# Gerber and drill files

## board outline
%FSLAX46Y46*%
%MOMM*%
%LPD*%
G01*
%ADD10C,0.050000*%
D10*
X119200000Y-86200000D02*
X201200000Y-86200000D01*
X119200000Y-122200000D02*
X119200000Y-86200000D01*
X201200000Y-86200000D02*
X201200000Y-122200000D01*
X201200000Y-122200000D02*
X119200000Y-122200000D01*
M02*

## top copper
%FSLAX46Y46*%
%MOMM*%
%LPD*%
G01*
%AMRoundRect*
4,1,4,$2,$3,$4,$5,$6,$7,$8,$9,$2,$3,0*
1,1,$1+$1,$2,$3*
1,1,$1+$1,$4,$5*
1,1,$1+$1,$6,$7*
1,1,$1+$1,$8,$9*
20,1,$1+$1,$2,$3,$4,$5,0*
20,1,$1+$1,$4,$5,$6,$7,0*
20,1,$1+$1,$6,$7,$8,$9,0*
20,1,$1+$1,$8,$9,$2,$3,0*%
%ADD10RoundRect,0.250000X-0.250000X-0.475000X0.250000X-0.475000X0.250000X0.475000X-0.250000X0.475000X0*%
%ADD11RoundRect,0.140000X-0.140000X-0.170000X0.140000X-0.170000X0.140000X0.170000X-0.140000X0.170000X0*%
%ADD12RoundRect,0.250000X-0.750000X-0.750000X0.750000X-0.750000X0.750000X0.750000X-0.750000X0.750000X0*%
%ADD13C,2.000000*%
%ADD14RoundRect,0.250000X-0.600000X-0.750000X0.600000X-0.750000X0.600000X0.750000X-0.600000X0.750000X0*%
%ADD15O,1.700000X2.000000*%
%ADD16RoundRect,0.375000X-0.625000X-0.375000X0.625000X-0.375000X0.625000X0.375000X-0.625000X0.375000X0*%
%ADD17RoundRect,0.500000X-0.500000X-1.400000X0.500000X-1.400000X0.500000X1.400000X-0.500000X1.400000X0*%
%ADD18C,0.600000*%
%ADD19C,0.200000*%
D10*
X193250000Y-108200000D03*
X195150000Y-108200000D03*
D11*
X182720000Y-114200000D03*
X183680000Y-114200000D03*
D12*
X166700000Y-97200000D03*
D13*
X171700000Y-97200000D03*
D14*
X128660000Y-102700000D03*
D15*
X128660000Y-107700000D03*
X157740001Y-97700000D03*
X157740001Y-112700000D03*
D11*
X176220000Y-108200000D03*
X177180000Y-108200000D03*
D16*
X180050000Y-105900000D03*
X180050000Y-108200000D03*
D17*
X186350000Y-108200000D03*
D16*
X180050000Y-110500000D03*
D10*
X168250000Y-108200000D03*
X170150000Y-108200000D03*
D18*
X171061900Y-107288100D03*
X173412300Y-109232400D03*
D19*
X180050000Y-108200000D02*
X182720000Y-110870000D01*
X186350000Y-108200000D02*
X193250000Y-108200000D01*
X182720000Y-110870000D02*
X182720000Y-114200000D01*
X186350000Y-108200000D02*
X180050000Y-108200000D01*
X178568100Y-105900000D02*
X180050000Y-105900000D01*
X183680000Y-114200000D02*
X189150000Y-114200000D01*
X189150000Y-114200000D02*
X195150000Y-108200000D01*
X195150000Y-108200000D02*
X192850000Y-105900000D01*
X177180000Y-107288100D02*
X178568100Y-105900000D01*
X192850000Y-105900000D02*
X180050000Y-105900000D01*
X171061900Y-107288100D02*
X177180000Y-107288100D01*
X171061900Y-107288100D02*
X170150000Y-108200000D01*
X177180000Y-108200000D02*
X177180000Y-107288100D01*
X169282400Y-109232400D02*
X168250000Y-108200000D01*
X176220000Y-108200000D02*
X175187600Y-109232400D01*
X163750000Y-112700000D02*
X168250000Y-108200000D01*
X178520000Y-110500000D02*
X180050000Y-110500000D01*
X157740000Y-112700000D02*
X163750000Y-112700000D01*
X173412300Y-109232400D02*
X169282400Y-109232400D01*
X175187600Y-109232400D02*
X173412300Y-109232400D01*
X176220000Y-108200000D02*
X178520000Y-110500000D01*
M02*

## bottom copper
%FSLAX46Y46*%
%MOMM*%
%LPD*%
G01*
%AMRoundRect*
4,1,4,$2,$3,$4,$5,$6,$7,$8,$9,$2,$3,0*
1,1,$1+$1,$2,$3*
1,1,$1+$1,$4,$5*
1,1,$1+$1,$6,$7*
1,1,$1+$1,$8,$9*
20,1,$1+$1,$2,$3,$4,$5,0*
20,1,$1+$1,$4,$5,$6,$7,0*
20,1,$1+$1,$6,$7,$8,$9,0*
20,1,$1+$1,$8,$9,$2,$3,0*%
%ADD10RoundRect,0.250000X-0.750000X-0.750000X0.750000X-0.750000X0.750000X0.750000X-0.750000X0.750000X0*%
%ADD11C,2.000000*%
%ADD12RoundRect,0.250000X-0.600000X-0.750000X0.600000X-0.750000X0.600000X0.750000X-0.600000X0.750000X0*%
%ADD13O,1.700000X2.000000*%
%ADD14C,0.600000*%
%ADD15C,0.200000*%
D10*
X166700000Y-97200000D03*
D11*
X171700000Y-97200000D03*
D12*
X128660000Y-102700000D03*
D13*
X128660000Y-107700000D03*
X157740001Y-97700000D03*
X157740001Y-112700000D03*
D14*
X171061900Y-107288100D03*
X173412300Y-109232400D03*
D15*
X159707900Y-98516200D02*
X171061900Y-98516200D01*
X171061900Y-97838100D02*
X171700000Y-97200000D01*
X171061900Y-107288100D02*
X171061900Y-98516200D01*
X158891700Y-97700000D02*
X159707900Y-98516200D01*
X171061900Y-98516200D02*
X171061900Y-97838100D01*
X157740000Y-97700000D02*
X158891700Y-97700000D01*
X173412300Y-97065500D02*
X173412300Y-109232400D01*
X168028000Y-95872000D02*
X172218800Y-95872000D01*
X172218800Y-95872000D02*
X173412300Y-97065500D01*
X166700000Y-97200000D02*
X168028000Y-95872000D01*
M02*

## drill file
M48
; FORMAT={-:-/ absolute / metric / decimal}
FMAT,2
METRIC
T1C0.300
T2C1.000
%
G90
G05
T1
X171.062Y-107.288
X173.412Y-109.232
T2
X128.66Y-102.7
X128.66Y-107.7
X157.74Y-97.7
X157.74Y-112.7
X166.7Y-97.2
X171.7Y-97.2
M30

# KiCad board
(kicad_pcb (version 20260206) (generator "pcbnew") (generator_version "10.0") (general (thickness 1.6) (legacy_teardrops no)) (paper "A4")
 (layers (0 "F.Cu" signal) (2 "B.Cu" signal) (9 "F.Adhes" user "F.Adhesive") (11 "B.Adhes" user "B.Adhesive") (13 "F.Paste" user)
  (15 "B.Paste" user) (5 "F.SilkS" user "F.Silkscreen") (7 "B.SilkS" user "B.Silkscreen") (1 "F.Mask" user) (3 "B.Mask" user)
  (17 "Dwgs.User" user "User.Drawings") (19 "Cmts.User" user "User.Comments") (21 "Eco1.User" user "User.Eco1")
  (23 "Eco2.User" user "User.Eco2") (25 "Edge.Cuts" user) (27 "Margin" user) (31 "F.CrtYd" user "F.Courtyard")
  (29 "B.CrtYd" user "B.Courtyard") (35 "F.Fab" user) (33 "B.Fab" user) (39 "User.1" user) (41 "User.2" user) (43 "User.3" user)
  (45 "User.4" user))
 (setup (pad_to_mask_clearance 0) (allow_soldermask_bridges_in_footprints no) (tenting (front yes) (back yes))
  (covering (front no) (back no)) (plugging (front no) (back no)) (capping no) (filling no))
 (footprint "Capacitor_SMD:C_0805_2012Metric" (layer "F.Cu") (at 194.2 108.2)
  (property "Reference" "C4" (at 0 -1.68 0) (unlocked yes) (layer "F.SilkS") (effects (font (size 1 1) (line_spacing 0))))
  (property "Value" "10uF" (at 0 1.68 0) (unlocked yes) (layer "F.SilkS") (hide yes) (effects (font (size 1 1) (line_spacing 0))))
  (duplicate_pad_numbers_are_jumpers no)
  (pad "1" smd roundrect (at -0.95 0) (size 1 1.45) (layers "F.Cu" "F.Mask" "F.Paste") (roundrect_rratio 0.25) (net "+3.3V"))
  (pad "2" smd roundrect (at 0.95 0) (size 1 1.45) (layers "F.Cu" "F.Mask" "F.Paste") (roundrect_rratio 0.25) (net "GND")))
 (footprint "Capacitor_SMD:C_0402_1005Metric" (layer "F.Cu") (at 183.2 114.2)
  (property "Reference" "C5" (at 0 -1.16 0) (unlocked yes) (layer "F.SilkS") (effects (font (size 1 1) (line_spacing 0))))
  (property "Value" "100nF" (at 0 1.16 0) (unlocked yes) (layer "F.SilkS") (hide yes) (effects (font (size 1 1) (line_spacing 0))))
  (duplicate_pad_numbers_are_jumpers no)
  (pad "1" smd roundrect (at -0.48 0) (size 0.56 0.62) (layers "F.Cu" "F.Mask" "F.Paste") (roundrect_rratio 0.25) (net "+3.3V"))
  (pad "2" smd roundrect (at 0.48 0) (size 0.56 0.62) (layers "F.Cu" "F.Mask" "F.Paste") (roundrect_rratio 0.25) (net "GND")))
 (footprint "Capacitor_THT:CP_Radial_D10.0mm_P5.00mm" (layer "F.Cu") (at 166.7 97.2)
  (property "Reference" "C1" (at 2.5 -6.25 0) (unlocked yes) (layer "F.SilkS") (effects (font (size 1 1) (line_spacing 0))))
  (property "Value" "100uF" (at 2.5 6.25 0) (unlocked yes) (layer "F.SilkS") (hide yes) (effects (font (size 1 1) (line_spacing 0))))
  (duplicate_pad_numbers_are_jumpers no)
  (pad "1" thru_hole roundrect (at 0 0) (size 2 2) (drill 1) (layers "*.Cu" "*.Mask") (remove_unused_layers no) (roundrect_rratio 0.125)
   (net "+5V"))
  (pad "2" thru_hole circle (at 5 0) (size 2 2) (drill 1) (layers "*.Cu" "*.Mask") (remove_unused_layers no) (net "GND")))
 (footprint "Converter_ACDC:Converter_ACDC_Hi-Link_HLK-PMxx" (layer "F.Cu") (at 128.66 102.7)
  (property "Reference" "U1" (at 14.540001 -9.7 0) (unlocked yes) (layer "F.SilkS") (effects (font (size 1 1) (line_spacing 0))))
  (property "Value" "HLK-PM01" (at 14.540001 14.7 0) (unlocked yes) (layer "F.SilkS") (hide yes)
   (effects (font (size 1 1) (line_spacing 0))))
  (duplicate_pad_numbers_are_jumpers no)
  (pad "1" thru_hole roundrect (at 0 0) (size 1.7 2) (drill 1) (layers "*.Cu" "*.Mask") (remove_unused_layers no)
   (roundrect_rratio 0.147059) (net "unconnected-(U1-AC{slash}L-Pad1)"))
  (pad "2" thru_hole oval (at 0 5) (size 1.7 2) (drill 1) (layers "*.Cu" "*.Mask") (remove_unused_layers no)
   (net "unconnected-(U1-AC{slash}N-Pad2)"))
  (pad "3" thru_hole oval (at 29.080001 -5) (size 1.7 2) (drill 1) (layers "*.Cu" "*.Mask") (remove_unused_layers no) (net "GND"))
  (pad "4" thru_hole oval (at 29.080001 10) (size 1.7 2) (drill 1) (layers "*.Cu" "*.Mask") (remove_unused_layers no) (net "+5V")))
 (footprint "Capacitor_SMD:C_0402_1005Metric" (layer "F.Cu") (at 176.7 108.2)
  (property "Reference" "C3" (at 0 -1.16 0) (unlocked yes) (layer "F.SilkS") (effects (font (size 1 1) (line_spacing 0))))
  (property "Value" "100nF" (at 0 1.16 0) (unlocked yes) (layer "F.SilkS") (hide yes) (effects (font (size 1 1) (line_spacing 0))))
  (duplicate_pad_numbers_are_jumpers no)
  (pad "1" smd roundrect (at -0.48 0) (size 0.56 0.62) (layers "F.Cu" "F.Mask" "F.Paste") (roundrect_rratio 0.25) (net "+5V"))
  (pad "2" smd roundrect (at 0.48 0) (size 0.56 0.62) (layers "F.Cu" "F.Mask" "F.Paste") (roundrect_rratio 0.25) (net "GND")))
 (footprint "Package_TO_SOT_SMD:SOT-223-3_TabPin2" (layer "F.Cu") (at 183.2 108.2)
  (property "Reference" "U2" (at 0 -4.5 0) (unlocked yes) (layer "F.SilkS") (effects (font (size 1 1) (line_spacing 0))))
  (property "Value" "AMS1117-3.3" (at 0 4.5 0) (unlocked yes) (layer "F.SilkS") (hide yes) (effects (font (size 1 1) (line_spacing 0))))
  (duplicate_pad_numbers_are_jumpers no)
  (pad "1" smd roundrect (at -3.15 -2.3) (size 2 1.5) (layers "F.Cu" "F.Mask" "F.Paste") (roundrect_rratio 0.25) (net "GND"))
  (pad "2" smd roundrect (at -3.15 0) (size 2 1.5) (layers "F.Cu" "F.Mask" "F.Paste") (roundrect_rratio 0.25) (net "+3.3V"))
  (pad "2" smd roundrect (at 3.15 0) (size 2 3.8) (layers "F.Cu" "F.Mask" "F.Paste") (roundrect_rratio 0.25) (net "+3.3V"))
  (pad "3" smd roundrect (at -3.15 2.3) (size 2 1.5) (layers "F.Cu" "F.Mask" "F.Paste") (roundrect_rratio 0.25) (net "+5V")))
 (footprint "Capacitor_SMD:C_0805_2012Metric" (layer "F.Cu") (at 169.2 108.2)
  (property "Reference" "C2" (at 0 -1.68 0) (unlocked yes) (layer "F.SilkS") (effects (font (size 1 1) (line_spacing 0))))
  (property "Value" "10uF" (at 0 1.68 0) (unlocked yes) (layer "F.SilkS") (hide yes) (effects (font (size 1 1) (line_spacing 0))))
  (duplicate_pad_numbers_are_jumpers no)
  (pad "1" smd roundrect (at -0.95 0) (size 1 1.45) (layers "F.Cu" "F.Mask" "F.Paste") (roundrect_rratio 0.25) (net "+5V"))
  (pad "2" smd roundrect (at 0.95 0) (size 1 1.45) (layers "F.Cu" "F.Mask" "F.Paste") (roundrect_rratio 0.25) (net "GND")))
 (gr_line (start 119.2 86.2) (end 201.2 86.2) (stroke (width 0.05) (type default)) (layer "Edge.Cuts"))
 (gr_line (start 119.2 122.2) (end 119.2 86.2) (stroke (width 0.05) (type default)) (layer "Edge.Cuts"))
 (gr_line (start 201.2 86.2) (end 201.2 122.2) (stroke (width 0.05) (type default)) (layer "Edge.Cuts"))
 (gr_line (start 201.2 122.2) (end 119.2 122.2) (stroke (width 0.05) (type default)) (layer "Edge.Cuts"))
 (segment (start 180.05 108.2) (end 182.72 110.87) (width 0.2) (layer "F.Cu") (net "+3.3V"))
 (segment (start 186.35 108.2) (end 193.25 108.2) (width 0.2) (layer "F.Cu") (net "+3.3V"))
 (segment (start 182.72 110.87) (end 182.72 114.2) (width 0.2) (layer "F.Cu") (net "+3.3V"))
 (segment (start 186.35 108.2) (end 180.05 108.2) (width 0.2) (layer "F.Cu") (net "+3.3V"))
 (segment (start 178.5681 105.9) (end 180.05 105.9) (width 0.2) (layer "F.Cu") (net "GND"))
 (segment (start 183.68 114.2) (end 189.15 114.2) (width 0.2) (layer "F.Cu") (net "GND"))
 (segment (start 189.15 114.2) (end 195.15 108.2) (width 0.2) (layer "F.Cu") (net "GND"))
 (segment (start 195.15 108.2) (end 192.85 105.9) (width 0.2) (layer "F.Cu") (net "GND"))
 (segment (start 177.18 107.2881) (end 178.5681 105.9) (width 0.2) (layer "F.Cu") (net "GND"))
 (segment (start 192.85 105.9) (end 180.05 105.9) (width 0.2) (layer "F.Cu") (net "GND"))
 (segment (start 171.0619 107.2881) (end 177.18 107.2881) (width 0.2) (layer "F.Cu") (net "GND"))
 (segment (start 171.0619 107.2881) (end 170.15 108.2) (width 0.2) (layer "F.Cu") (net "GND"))
 (segment (start 177.18 108.2) (end 177.18 107.2881) (width 0.2) (layer "F.Cu") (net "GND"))
 (via (at 171.0619 107.2881) (size 0.6) (drill 0.3) (layers "F.Cu" "B.Cu") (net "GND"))
 (segment (start 159.7079 98.5162) (end 171.0619 98.5162) (width 0.2) (layer "B.Cu") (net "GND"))
 (segment (start 171.0619 97.8381) (end 171.7 97.2) (width 0.2) (layer "B.Cu") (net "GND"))
 (segment (start 171.0619 107.2881) (end 171.0619 98.5162) (width 0.2) (layer "B.Cu") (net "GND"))
 (segment (start 158.8917 97.7) (end 159.7079 98.5162) (width 0.2) (layer "B.Cu") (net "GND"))
 (segment (start 171.0619 98.5162) (end 171.0619 97.8381) (width 0.2) (layer "B.Cu") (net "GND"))
 (segment (start 157.74 97.7) (end 158.8917 97.7) (width 0.2) (layer "B.Cu") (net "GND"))
 (segment (start 169.2824 109.2324) (end 168.25 108.2) (width 0.2) (layer "F.Cu") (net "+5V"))
 (segment (start 176.22 108.2) (end 175.1876 109.2324) (width 0.2) (layer "F.Cu") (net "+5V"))
 (segment (start 163.75 112.7) (end 168.25 108.2) (width 0.2) (layer "F.Cu") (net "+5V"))
 (segment (start 178.52 110.5) (end 180.05 110.5) (width 0.2) (layer "F.Cu") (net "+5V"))
 (segment (start 157.74 112.7) (end 163.75 112.7) (width 0.2) (layer "F.Cu") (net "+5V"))
 (segment (start 173.4123 109.2324) (end 169.2824 109.2324) (width 0.2) (layer "F.Cu") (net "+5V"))
 (segment (start 175.1876 109.2324) (end 173.4123 109.2324) (width 0.2) (layer "F.Cu") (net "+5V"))
 (segment (start 176.22 108.2) (end 178.52 110.5) (width 0.2) (layer "F.Cu") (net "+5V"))
 (via (at 173.4123 109.2324) (size 0.6) (drill 0.3) (layers "F.Cu" "B.Cu") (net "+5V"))
 (segment (start 173.4123 97.0655) (end 173.4123 109.2324) (width 0.2) (layer "B.Cu") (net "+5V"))
 (segment (start 168.028 95.872) (end 172.2188 95.872) (width 0.2) (layer "B.Cu") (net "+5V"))
 (segment (start 172.2188 95.872) (end 173.4123 97.0655) (width 0.2) (layer "B.Cu") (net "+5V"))
 (segment (start 166.7 97.2) (end 168.028 95.872) (width 0.2) (layer "B.Cu") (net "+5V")))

